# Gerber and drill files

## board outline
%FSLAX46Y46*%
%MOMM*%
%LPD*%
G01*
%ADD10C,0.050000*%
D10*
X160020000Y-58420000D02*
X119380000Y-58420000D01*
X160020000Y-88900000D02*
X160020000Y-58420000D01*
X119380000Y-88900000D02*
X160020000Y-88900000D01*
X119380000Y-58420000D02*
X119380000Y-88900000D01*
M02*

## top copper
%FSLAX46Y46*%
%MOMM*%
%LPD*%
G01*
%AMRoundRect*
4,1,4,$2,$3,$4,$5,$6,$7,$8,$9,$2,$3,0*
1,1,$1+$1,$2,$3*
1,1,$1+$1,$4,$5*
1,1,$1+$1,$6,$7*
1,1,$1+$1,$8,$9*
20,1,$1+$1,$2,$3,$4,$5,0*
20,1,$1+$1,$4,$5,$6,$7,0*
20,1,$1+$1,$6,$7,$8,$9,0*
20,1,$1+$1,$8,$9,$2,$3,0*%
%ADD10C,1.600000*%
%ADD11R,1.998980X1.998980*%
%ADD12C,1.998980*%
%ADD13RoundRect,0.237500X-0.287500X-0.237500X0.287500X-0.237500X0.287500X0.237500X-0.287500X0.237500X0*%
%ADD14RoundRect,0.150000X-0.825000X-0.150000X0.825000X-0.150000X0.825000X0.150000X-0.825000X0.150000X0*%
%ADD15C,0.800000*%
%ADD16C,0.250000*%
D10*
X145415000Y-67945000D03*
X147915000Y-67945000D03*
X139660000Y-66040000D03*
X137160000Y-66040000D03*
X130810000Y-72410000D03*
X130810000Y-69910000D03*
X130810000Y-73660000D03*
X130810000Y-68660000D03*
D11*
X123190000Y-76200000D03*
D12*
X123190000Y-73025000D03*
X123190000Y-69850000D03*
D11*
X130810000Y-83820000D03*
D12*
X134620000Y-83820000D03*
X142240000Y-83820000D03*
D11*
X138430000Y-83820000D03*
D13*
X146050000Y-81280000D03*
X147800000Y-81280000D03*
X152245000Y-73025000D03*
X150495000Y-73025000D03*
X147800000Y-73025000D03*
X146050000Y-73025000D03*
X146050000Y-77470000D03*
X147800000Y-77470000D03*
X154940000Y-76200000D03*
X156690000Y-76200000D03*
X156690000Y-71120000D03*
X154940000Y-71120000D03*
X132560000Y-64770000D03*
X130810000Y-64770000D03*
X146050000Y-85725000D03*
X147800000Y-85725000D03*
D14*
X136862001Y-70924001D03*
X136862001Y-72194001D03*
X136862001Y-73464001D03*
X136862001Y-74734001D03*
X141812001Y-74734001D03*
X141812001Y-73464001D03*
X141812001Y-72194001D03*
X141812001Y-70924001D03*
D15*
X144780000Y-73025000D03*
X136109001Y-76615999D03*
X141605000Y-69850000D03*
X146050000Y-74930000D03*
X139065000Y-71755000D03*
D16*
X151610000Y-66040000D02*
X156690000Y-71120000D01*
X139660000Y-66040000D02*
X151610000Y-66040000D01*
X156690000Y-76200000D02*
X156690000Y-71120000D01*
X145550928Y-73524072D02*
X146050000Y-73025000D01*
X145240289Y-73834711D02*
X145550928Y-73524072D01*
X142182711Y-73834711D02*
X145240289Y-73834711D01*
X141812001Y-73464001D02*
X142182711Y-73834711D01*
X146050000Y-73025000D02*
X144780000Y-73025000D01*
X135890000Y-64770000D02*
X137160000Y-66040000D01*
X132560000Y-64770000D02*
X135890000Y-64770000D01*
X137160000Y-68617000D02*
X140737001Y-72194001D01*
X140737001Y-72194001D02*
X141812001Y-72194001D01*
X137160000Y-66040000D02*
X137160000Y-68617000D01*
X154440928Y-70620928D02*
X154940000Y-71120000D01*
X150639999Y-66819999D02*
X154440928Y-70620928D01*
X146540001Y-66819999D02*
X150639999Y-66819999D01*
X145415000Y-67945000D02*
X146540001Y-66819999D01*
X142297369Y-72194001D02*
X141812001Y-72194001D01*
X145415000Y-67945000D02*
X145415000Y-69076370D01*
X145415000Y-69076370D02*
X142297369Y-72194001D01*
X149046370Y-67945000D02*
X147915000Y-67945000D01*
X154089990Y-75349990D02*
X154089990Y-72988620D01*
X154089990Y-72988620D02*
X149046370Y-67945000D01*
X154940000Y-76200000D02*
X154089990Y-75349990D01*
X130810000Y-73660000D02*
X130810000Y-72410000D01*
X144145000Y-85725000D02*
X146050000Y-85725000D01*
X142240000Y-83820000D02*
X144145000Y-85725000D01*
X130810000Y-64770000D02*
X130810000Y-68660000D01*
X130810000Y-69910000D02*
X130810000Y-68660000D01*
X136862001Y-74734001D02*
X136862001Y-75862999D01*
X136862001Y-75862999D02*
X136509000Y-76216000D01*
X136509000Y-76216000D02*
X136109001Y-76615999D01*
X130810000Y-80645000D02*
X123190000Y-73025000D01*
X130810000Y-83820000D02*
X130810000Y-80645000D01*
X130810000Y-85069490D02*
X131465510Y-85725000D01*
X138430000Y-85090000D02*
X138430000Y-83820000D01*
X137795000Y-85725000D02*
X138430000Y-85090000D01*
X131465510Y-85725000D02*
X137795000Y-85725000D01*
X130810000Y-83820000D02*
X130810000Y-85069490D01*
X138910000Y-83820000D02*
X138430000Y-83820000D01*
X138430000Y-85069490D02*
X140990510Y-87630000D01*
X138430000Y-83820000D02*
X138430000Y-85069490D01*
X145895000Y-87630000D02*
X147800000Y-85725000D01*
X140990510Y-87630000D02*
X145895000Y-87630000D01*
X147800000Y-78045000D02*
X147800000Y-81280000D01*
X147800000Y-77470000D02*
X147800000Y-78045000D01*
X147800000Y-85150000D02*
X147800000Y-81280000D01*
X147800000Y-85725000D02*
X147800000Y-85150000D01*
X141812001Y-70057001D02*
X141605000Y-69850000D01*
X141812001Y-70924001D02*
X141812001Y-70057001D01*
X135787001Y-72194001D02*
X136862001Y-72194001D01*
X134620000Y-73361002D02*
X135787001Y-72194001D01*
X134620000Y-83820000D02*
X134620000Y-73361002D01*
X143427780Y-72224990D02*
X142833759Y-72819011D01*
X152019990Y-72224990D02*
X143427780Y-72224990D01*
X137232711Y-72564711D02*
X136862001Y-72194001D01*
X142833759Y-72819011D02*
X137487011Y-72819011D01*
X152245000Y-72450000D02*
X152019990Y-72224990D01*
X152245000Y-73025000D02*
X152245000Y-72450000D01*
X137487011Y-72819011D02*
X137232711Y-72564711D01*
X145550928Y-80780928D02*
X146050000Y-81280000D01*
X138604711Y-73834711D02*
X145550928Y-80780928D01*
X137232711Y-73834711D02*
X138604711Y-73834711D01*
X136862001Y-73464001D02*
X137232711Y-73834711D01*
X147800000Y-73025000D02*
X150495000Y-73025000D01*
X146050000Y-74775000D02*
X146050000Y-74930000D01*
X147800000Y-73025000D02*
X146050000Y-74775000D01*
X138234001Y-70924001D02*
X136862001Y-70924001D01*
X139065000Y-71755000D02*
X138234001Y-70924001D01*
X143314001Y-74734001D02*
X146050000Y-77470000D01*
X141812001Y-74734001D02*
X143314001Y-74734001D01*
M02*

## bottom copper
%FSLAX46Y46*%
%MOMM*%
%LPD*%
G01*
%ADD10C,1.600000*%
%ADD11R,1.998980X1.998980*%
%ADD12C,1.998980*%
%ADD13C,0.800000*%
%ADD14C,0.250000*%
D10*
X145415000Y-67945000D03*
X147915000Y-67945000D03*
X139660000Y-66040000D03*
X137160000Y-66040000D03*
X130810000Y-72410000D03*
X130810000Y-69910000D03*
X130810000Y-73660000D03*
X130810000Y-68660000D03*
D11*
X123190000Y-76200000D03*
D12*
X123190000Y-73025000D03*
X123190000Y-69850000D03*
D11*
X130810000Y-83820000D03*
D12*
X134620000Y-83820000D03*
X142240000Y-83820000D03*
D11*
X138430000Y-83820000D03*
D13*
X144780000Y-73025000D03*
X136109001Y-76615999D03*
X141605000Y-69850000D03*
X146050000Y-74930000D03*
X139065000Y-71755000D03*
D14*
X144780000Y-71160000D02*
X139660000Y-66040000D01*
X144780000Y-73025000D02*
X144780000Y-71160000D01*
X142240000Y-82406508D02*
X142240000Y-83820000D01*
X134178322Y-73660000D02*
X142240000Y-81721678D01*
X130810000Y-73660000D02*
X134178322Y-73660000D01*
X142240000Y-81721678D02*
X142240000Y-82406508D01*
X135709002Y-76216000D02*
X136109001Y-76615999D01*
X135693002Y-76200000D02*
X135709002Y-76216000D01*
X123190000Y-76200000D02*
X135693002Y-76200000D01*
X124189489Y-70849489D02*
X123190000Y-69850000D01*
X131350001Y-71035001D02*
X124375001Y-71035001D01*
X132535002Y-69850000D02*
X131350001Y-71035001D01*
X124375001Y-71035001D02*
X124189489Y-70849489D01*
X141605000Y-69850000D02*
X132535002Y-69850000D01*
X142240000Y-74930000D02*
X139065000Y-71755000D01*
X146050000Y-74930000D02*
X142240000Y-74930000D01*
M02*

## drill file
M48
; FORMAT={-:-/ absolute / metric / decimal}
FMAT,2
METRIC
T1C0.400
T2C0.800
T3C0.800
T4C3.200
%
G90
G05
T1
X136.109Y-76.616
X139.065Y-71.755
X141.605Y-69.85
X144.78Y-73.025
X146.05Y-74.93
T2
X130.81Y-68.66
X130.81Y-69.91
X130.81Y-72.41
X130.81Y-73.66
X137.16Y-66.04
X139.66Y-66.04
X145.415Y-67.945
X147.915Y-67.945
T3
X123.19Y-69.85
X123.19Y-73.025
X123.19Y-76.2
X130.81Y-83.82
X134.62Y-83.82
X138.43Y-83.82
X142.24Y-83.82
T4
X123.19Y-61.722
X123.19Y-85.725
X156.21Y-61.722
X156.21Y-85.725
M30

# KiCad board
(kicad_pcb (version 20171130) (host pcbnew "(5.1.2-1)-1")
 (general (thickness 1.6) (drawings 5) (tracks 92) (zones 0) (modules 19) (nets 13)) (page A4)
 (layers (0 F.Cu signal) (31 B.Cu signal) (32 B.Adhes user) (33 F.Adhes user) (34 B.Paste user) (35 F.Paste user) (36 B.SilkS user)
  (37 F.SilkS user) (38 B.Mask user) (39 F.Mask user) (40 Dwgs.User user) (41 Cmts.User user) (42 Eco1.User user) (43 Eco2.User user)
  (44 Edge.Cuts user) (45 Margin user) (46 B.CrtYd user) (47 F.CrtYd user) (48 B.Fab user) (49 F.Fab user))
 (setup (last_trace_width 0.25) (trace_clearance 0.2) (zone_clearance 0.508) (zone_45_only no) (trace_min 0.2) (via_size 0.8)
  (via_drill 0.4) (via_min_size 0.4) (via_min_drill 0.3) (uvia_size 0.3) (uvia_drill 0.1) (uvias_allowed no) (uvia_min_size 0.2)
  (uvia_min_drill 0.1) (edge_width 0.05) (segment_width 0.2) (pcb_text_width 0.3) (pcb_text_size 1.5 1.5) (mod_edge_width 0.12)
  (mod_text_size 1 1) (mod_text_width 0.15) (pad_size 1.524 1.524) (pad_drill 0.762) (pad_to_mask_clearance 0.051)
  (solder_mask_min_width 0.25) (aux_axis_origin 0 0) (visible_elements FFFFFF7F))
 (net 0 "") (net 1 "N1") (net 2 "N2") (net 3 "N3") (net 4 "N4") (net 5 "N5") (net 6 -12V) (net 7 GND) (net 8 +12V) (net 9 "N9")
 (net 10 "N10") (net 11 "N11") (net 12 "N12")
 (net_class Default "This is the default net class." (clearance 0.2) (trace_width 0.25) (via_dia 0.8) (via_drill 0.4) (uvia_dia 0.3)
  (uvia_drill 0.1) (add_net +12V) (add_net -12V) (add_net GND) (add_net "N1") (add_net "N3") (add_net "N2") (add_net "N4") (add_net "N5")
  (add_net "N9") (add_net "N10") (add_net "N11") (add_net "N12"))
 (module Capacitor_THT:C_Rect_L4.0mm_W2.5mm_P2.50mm (layer F.Cu) (at 145.415 67.945)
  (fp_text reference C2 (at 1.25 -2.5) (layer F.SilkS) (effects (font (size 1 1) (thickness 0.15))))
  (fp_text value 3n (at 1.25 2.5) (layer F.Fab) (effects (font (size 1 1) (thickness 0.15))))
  (pad 1 thru_hole circle (at 0 0) (size 1.6 1.6) (drill 0.8) (layers *.Cu *.Mask) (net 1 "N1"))
  (pad 2 thru_hole circle (at 2.5 0) (size 1.6 1.6) (drill 0.8) (layers *.Cu *.Mask) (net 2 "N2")))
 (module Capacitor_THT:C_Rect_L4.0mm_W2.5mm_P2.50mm (layer F.Cu) (at 137.16 66.04)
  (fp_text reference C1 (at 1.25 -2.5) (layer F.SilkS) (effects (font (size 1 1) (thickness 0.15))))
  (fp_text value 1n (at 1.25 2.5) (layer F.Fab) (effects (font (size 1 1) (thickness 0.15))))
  (pad 2 thru_hole circle (at 2.5 0) (size 1.6 1.6) (drill 0.8) (layers *.Cu *.Mask) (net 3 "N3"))
  (pad 1 thru_hole circle (at 0 0) (size 1.6 1.6) (drill 0.8) (layers *.Cu *.Mask) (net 1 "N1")))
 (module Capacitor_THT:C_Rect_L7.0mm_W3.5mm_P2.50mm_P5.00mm (layer F.Cu) (at 130.81 73.66 90)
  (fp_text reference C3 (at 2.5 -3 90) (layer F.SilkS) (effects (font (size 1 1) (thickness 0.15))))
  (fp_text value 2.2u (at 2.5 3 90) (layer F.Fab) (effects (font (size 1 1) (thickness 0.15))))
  (pad 1 thru_hole circle (at 1.25 0 90) (size 1.6 1.6) (drill 0.8) (layers *.Cu *.Mask) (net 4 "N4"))
  (pad 2 thru_hole circle (at 3.75 0 90) (size 1.6 1.6) (drill 0.8) (layers *.Cu *.Mask) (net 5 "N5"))
  (pad 1 thru_hole circle (at 0 0 90) (size 1.6 1.6) (drill 0.8) (layers *.Cu *.Mask) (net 4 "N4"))
  (pad 2 thru_hole circle (at 5 0 90) (size 1.6 1.6) (drill 0.8) (layers *.Cu *.Mask) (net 5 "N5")))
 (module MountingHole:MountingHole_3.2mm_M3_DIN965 (layer F.Cu) (at 123.19 61.722)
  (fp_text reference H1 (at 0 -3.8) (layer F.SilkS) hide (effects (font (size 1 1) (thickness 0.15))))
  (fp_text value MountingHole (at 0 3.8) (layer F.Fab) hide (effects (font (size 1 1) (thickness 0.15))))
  (pad 1 np_thru_hole circle (at 0 0) (size 3.2 3.2) (drill 3.2) (layers *.Cu *.Mask)))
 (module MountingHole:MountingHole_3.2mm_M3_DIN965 (layer F.Cu) (at 123.19 85.725)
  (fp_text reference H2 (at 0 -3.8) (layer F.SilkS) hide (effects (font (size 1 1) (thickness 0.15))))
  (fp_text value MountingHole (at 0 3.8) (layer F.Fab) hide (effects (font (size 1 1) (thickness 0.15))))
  (pad 1 np_thru_hole circle (at 0 0) (size 3.2 3.2) (drill 3.2) (layers *.Cu *.Mask)))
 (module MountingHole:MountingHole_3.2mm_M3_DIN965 (layer F.Cu) (at 156.21 85.725)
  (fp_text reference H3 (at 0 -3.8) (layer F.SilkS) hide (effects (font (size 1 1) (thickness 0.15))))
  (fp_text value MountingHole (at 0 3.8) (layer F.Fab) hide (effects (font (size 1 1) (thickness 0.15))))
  (pad 1 np_thru_hole circle (at 0 0) (size 3.2 3.2) (drill 3.2) (layers *.Cu *.Mask)))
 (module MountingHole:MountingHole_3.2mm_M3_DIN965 (layer F.Cu) (at 156.21 61.722)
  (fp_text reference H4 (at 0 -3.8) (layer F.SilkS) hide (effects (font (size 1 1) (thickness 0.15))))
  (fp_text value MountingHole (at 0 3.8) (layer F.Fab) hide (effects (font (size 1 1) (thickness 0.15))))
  (pad 1 np_thru_hole circle (at 0 0) (size 3.2 3.2) (drill 3.2) (layers *.Cu *.Mask)))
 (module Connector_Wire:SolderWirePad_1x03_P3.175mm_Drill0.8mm (layer F.Cu) (at 123.19 76.2 90)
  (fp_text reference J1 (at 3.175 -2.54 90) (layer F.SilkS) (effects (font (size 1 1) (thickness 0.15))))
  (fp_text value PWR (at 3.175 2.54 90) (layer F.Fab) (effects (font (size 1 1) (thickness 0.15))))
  (pad 1 thru_hole rect (at 0 0 90) (size 1.99898 1.99898) (drill 0.8001) (layers *.Cu *.Mask) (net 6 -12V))
  (pad 2 thru_hole circle (at 3.175 0 90) (size 1.99898 1.99898) (drill 0.8001) (layers *.Cu *.Mask) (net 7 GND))
  (pad 3 thru_hole circle (at 6.35 0 90) (size 1.99898 1.99898) (drill 0.8001) (layers *.Cu *.Mask) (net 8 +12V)))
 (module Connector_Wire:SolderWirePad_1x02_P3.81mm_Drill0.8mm (layer F.Cu) (at 130.81 83.82)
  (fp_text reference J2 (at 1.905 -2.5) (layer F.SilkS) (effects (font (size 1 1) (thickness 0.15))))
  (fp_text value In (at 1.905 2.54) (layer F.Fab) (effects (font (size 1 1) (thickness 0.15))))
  (pad 1 thru_hole rect (at 0 0) (size 1.99898 1.99898) (drill 0.8001) (layers *.Cu *.Mask) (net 7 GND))
  (pad 2 thru_hole circle (at 3.81 0) (size 1.99898 1.99898) (drill 0.8001) (layers *.Cu *.Mask) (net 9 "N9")))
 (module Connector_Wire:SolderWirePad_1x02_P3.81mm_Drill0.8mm (layer F.Cu) (at 138.43 83.82)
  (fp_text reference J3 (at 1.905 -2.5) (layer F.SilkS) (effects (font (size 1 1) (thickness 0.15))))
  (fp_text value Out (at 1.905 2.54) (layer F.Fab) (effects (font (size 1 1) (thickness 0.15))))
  (pad 2 thru_hole circle (at 3.81 0) (size 1.99898 1.99898) (drill 0.8001) (layers *.Cu *.Mask) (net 4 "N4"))
  (pad 1 thru_hole rect (at 0 0) (size 1.99898 1.99898) (drill 0.8001) (layers *.Cu *.Mask) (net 7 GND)))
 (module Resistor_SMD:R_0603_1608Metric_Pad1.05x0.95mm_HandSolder (layer F.Cu) (at 146.925 81.28)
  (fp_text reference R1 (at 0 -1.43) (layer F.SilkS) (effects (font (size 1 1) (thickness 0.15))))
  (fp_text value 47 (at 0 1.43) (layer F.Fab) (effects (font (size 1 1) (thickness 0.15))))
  (pad 1 smd roundrect (at -0.875 0) (size 1.05 0.95) (layers F.Cu F.Paste F.Mask) (roundrect_rratio 0.25) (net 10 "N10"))
  (pad 2 smd roundrect (at 0.875 0) (size 1.05 0.95) (layers F.Cu F.Paste F.Mask) (roundrect_rratio 0.25) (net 7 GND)))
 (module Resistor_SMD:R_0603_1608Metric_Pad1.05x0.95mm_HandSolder (layer F.Cu) (at 151.37 73.025)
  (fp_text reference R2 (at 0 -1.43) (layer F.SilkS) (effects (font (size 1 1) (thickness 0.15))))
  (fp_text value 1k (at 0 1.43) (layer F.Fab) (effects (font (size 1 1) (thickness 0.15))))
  (pad 2 smd roundrect (at 0.875 0) (size 1.05 0.95) (layers F.Cu F.Paste F.Mask) (roundrect_rratio 0.25) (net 9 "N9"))
  (pad 1 smd roundrect (at -0.875 0) (size 1.05 0.95) (layers F.Cu F.Paste F.Mask) (roundrect_rratio 0.25) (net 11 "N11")))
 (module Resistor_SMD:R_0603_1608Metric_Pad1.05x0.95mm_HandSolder (layer F.Cu) (at 146.925 73.025)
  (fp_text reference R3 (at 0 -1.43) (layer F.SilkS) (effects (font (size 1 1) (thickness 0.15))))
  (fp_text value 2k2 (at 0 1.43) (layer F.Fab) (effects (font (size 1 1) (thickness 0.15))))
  (pad 2 smd roundrect (at 0.875 0) (size 1.05 0.95) (layers F.Cu F.Paste F.Mask) (roundrect_rratio 0.25) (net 11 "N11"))
  (pad 1 smd roundrect (at -0.875 0) (size 1.05 0.95) (layers F.Cu F.Paste F.Mask) (roundrect_rratio 0.25) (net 3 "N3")))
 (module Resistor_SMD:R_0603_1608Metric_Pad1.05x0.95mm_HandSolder (layer F.Cu) (at 146.925 77.47)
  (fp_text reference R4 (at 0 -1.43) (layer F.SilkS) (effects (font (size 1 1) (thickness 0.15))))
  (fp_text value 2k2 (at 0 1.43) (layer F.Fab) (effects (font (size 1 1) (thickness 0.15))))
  (pad 1 smd roundrect (at -0.875 0) (size 1.05 0.95) (layers F.Cu F.Paste F.Mask) (roundrect_rratio 0.25) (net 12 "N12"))
  (pad 2 smd roundrect (at 0.875 0) (size 1.05 0.95) (layers F.Cu F.Paste F.Mask) (roundrect_rratio 0.25) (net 7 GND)))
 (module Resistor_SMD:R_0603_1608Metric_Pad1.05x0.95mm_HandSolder (layer F.Cu) (at 155.815 76.2)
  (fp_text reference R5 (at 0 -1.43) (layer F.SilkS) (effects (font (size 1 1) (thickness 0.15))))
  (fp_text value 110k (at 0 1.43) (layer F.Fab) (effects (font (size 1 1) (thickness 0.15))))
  (pad 1 smd roundrect (at -0.875 0) (size 1.05 0.95) (layers F.Cu F.Paste F.Mask) (roundrect_rratio 0.25) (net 2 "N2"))
  (pad 2 smd roundrect (at 0.875 0) (size 1.05 0.95) (layers F.Cu F.Paste F.Mask) (roundrect_rratio 0.25) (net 3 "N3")))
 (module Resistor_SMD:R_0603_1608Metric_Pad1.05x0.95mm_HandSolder (layer F.Cu) (at 155.815 71.12)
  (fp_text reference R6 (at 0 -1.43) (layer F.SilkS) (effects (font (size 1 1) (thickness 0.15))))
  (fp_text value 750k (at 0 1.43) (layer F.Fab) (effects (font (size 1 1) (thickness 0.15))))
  (pad 2 smd roundrect (at 0.875 0) (size 1.05 0.95) (layers F.Cu F.Paste F.Mask) (roundrect_rratio 0.25) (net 3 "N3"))
  (pad 1 smd roundrect (at -0.875 0) (size 1.05 0.95) (layers F.Cu F.Paste F.Mask) (roundrect_rratio 0.25) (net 1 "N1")))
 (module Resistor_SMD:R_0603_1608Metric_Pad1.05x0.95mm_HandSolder (layer F.Cu) (at 131.685 64.77)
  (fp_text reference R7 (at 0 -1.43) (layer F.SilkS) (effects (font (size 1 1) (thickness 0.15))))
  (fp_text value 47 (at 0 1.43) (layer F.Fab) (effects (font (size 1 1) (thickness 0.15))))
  (pad 2 smd roundrect (at 0.875 0) (size 1.05 0.95) (layers F.Cu F.Paste F.Mask) (roundrect_rratio 0.25) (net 1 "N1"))
  (pad 1 smd roundrect (at -0.875 0) (size 1.05 0.95) (layers F.Cu F.Paste F.Mask) (roundrect_rratio 0.25) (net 5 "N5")))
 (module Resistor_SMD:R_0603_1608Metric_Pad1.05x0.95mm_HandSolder (layer F.Cu) (at 146.925 85.725)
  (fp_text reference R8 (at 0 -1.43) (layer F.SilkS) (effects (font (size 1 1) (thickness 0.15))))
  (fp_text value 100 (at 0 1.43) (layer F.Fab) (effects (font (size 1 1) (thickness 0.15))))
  (pad 1 smd roundrect (at -0.875 0) (size 1.05 0.95) (layers F.Cu F.Paste F.Mask) (roundrect_rratio 0.25) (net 4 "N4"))
  (pad 2 smd roundrect (at 0.875 0) (size 1.05 0.95) (layers F.Cu F.Paste F.Mask) (roundrect_rratio 0.25) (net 7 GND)))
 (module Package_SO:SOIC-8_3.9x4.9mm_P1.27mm (layer F.Cu) (at 139.337001 72.829001)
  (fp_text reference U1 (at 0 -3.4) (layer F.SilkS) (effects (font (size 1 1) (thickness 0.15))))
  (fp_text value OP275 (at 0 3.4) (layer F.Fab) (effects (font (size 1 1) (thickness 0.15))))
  (pad 1 smd roundrect (at -2.475 -1.905) (size 1.95 0.6) (layers F.Cu F.Paste F.Mask) (roundrect_rratio 0.25) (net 11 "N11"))
  (pad 2 smd roundrect (at -2.475 -0.635) (size 1.95 0.6) (layers F.Cu F.Paste F.Mask) (roundrect_rratio 0.25) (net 9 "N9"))
  (pad 3 smd roundrect (at -2.475 0.635) (size 1.95 0.6) (layers F.Cu F.Paste F.Mask) (roundrect_rratio 0.25) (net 10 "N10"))
  (pad 4 smd roundrect (at -2.475 1.905) (size 1.95 0.6) (layers F.Cu F.Paste F.Mask) (roundrect_rratio 0.25) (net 6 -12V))
  (pad 5 smd roundrect (at 2.475 1.905) (size 1.95 0.6) (layers F.Cu F.Paste F.Mask) (roundrect_rratio 0.25) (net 12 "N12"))
  (pad 6 smd roundrect (at 2.475 0.635) (size 1.95 0.6) (layers F.Cu F.Paste F.Mask) (roundrect_rratio 0.25) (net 3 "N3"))
  (pad 7 smd roundrect (at 2.475 -0.635) (size 1.95 0.6) (layers F.Cu F.Paste F.Mask) (roundrect_rratio 0.25) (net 1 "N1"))
  (pad 8 smd roundrect (at 2.475 -1.905) (size 1.95 0.6) (layers F.Cu F.Paste F.Mask) (roundrect_rratio 0.25) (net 8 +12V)))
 (gr_line (start 160.02 58.42) (end 119.38 58.42) (layer Edge.Cuts) (width 0.05))
 (gr_line (start 160.02 88.9) (end 160.02 58.42) (layer Edge.Cuts) (width 0.05))
 (gr_line (start 119.38 88.9) (end 160.02 88.9) (layer Edge.Cuts) (width 0.05))
 (gr_line (start 119.38 58.42) (end 119.38 88.9) (layer Edge.Cuts) (width 0.05))
 (segment (start 151.61 66.04) (end 156.69 71.12) (width 0.25) (layer F.Cu) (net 3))
 (segment (start 139.66 66.04) (end 151.61 66.04) (width 0.25) (layer F.Cu) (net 3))
 (segment (start 156.69 76.2) (end 156.69 71.12) (width 0.25) (layer F.Cu) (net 3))
 (segment (start 145.550928 73.524072) (end 146.05 73.025) (width 0.25) (layer F.Cu) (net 3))
 (segment (start 145.240289 73.834711) (end 145.550928 73.524072) (width 0.25) (layer F.Cu) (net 3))
 (segment (start 142.182711 73.834711) (end 145.240289 73.834711) (width 0.25) (layer F.Cu) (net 3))
 (segment (start 141.812001 73.464001) (end 142.182711 73.834711) (width 0.25) (layer F.Cu) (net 3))
 (via (at 144.78 73.025) (size 0.8) (drill 0.4) (layers F.Cu B.Cu) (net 3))
 (segment (start 146.05 73.025) (end 144.78 73.025) (width 0.25) (layer F.Cu) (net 3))
 (segment (start 144.78 71.16) (end 139.66 66.04) (width 0.25) (layer B.Cu) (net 3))
 (segment (start 144.78 73.025) (end 144.78 71.16) (width 0.25) (layer B.Cu) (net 3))
 (segment (start 135.89 64.77) (end 137.16 66.04) (width 0.25) (layer F.Cu) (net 1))
 (segment (start 132.56 64.77) (end 135.89 64.77) (width 0.25) (layer F.Cu) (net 1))
 (segment (start 137.16 68.617) (end 140.737001 72.194001) (width 0.25) (layer F.Cu) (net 1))
 (segment (start 140.737001 72.194001) (end 141.812001 72.194001) (width 0.25) (layer F.Cu) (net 1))
 (segment (start 137.16 66.04) (end 137.16 68.617) (width 0.25) (layer F.Cu) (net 1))
 (segment (start 154.440928 70.620928) (end 154.94 71.12) (width 0.25) (layer F.Cu) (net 1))
 (segment (start 150.639999 66.819999) (end 154.440928 70.620928) (width 0.25) (layer F.Cu) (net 1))
 (segment (start 146.540001 66.819999) (end 150.639999 66.819999) (width 0.25) (layer F.Cu) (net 1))
 (segment (start 145.415 67.945) (end 146.540001 66.819999) (width 0.25) (layer F.Cu) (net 1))
 (segment (start 142.297369 72.194001) (end 141.812001 72.194001) (width 0.25) (layer F.Cu) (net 1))
 (segment (start 145.415 67.945) (end 145.415 69.07637) (width 0.25) (layer F.Cu) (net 1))
 (segment (start 145.415 69.07637) (end 142.297369 72.194001) (width 0.25) (layer F.Cu) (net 1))
 (segment (start 149.04637 67.945) (end 147.915 67.945) (width 0.25) (layer F.Cu) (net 2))
 (segment (start 154.08999 75.34999) (end 154.08999 72.98862) (width 0.25) (layer F.Cu) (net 2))
 (segment (start 154.08999 72.98862) (end 149.04637 67.945) (width 0.25) (layer F.Cu) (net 2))
 (segment (start 154.94 76.2) (end 154.08999 75.34999) (width 0.25) (layer F.Cu) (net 2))
 (segment (start 130.81 73.66) (end 130.81 72.41) (width 0.25) (layer F.Cu) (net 4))
 (segment (start 144.145 85.725) (end 146.05 85.725) (width 0.25) (layer F.Cu) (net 4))
 (segment (start 142.24 83.82) (end 144.145 85.725) (width 0.25) (layer F.Cu) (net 4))
 (segment (start 142.24 82.406508) (end 142.24 83.82) (width 0.25) (layer B.Cu) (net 4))
 (segment (start 134.178322 73.66) (end 142.24 81.721678) (width 0.25) (layer B.Cu) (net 4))
 (segment (start 130.81 73.66) (end 134.178322 73.66) (width 0.25) (layer B.Cu) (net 4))
 (segment (start 142.24 81.721678) (end 142.24 82.406508) (width 0.25) (layer B.Cu) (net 4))
 (segment (start 130.81 64.77) (end 130.81 68.66) (width 0.25) (layer F.Cu) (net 5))
 (segment (start 130.81 69.91) (end 130.81 68.66) (width 0.25) (layer F.Cu) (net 5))
 (via (at 136.109001 76.615999) (size 0.8) (drill 0.4) (layers F.Cu B.Cu) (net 6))
 (segment (start 136.862001 74.734001) (end 136.862001 75.862999) (width 0.25) (layer F.Cu) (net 6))
 (segment (start 136.862001 75.862999) (end 136.509 76.216) (width 0.25) (layer F.Cu) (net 6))
 (segment (start 136.509 76.216) (end 136.109001 76.615999) (width 0.25) (layer F.Cu) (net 6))
 (segment (start 135.709002 76.216) (end 136.109001 76.615999) (width 0.25) (layer B.Cu) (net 6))
 (segment (start 135.693002 76.2) (end 135.709002 76.216) (width 0.25) (layer B.Cu) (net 6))
 (segment (start 123.19 76.2) (end 135.693002 76.2) (width 0.25) (layer B.Cu) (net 6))
 (segment (start 130.81 80.645) (end 123.19 73.025) (width 0.25) (layer F.Cu) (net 7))
 (segment (start 130.81 83.82) (end 130.81 80.645) (width 0.25) (layer F.Cu) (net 7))
 (segment (start 130.81 85.06949) (end 131.46551 85.725) (width 0.25) (layer F.Cu) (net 7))
 (segment (start 138.43 85.09) (end 138.43 83.82) (width 0.25) (layer F.Cu) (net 7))
 (segment (start 137.795 85.725) (end 138.43 85.09) (width 0.25) (layer F.Cu) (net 7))
 (segment (start 131.46551 85.725) (end 137.795 85.725) (width 0.25) (layer F.Cu) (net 7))
 (segment (start 130.81 83.82) (end 130.81 85.06949) (width 0.25) (layer F.Cu) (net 7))
 (segment (start 138.91 83.82) (end 138.43 83.82) (width 0.25) (layer F.Cu) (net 7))
 (segment (start 138.43 85.06949) (end 140.99051 87.63) (width 0.25) (layer F.Cu) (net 7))
 (segment (start 138.43 83.82) (end 138.43 85.06949) (width 0.25) (layer F.Cu) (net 7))
 (segment (start 145.895 87.63) (end 147.8 85.725) (width 0.25) (layer F.Cu) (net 7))
 (segment (start 140.99051 87.63) (end 145.895 87.63) (width 0.25) (layer F.Cu) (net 7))
 (segment (start 147.8 78.045) (end 147.8 81.28) (width 0.25) (layer F.Cu) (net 7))
 (segment (start 147.8 77.47) (end 147.8 78.045) (width 0.25) (layer F.Cu) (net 7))
 (segment (start 147.8 85.15) (end 147.8 81.28) (width 0.25) (layer F.Cu) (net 7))
 (segment (start 147.8 85.725) (end 147.8 85.15) (width 0.25) (layer F.Cu) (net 7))
 (via (at 141.605 69.85) (size 0.8) (drill 0.4) (layers F.Cu B.Cu) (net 8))
 (segment (start 141.812001 70.057001) (end 141.605 69.85) (width 0.25) (layer F.Cu) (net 8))
 (segment (start 141.812001 70.924001) (end 141.812001 70.057001) (width 0.25) (layer F.Cu) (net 8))
 (segment (start 124.189489 70.849489) (end 123.19 69.85) (width 0.25) (layer B.Cu) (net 8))
 (segment (start 131.350001 71.035001) (end 124.375001 71.035001) (width 0.25) (layer B.Cu) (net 8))
 (segment (start 132.535002 69.85) (end 131.350001 71.035001) (width 0.25) (layer B.Cu) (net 8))
 (segment (start 124.375001 71.035001) (end 124.189489 70.849489) (width 0.25) (layer B.Cu) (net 8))
 (segment (start 141.605 69.85) (end 132.535002 69.85) (width 0.25) (layer B.Cu) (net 8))
 (segment (start 135.787001 72.194001) (end 136.862001 72.194001) (width 0.25) (layer F.Cu) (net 9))
 (segment (start 134.62 73.361002) (end 135.787001 72.194001) (width 0.25) (layer F.Cu) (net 9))
 (segment (start 134.62 83.82) (end 134.62 73.361002) (width 0.25) (layer F.Cu) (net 9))
 (segment (start 143.42778 72.22499) (end 142.833759 72.819011) (width 0.25) (layer F.Cu) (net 9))
 (segment (start 152.01999 72.22499) (end 143.42778 72.22499) (width 0.25) (layer F.Cu) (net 9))
 (segment (start 137.232711 72.564711) (end 136.862001 72.194001) (width 0.25) (layer F.Cu) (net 9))
 (segment (start 142.833759 72.819011) (end 137.487011 72.819011) (width 0.25) (layer F.Cu) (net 9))
 (segment (start 152.245 72.45) (end 152.01999 72.22499) (width 0.25) (layer F.Cu) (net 9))
 (segment (start 152.245 73.025) (end 152.245 72.45) (width 0.25) (layer F.Cu) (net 9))
 (segment (start 137.487011 72.819011) (end 137.232711 72.564711) (width 0.25) (layer F.Cu) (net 9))
 (segment (start 145.550928 80.780928) (end 146.05 81.28) (width 0.25) (layer F.Cu) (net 10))
 (segment (start 138.604711 73.834711) (end 145.550928 80.780928) (width 0.25) (layer F.Cu) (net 10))
 (segment (start 137.232711 73.834711) (end 138.604711 73.834711) (width 0.25) (layer F.Cu) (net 10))
 (segment (start 136.862001 73.464001) (end 137.232711 73.834711) (width 0.25) (layer F.Cu) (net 10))
 (segment (start 147.8 73.025) (end 150.495 73.025) (width 0.25) (layer F.Cu) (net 11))
 (via (at 146.05 74.93) (size 0.8) (drill 0.4) (layers F.Cu B.Cu) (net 11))
 (segment (start 146.05 74.775) (end 146.05 74.93) (width 0.25) (layer F.Cu) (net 11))
 (segment (start 147.8 73.025) (end 146.05 74.775) (width 0.25) (layer F.Cu) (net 11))
 (via (at 139.065 71.755) (size 0.8) (drill 0.4) (layers F.Cu B.Cu) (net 11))
 (segment (start 142.24 74.93) (end 139.065 71.755) (width 0.25) (layer B.Cu) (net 11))
 (segment (start 146.05 74.93) (end 142.24 74.93) (width 0.25) (layer B.Cu) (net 11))
 (segment (start 138.234001 70.924001) (end 136.862001 70.924001) (width 0.25) (layer F.Cu) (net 11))
 (segment (start 139.065 71.755) (end 138.234001 70.924001) (width 0.25) (layer F.Cu) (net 11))
 (segment (start 143.314001 74.734001) (end 146.05 77.47) (width 0.25) (layer F.Cu) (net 12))
 (segment (start 141.812001 74.734001) (end 143.314001 74.734001) (width 0.25) (layer F.Cu) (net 12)))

